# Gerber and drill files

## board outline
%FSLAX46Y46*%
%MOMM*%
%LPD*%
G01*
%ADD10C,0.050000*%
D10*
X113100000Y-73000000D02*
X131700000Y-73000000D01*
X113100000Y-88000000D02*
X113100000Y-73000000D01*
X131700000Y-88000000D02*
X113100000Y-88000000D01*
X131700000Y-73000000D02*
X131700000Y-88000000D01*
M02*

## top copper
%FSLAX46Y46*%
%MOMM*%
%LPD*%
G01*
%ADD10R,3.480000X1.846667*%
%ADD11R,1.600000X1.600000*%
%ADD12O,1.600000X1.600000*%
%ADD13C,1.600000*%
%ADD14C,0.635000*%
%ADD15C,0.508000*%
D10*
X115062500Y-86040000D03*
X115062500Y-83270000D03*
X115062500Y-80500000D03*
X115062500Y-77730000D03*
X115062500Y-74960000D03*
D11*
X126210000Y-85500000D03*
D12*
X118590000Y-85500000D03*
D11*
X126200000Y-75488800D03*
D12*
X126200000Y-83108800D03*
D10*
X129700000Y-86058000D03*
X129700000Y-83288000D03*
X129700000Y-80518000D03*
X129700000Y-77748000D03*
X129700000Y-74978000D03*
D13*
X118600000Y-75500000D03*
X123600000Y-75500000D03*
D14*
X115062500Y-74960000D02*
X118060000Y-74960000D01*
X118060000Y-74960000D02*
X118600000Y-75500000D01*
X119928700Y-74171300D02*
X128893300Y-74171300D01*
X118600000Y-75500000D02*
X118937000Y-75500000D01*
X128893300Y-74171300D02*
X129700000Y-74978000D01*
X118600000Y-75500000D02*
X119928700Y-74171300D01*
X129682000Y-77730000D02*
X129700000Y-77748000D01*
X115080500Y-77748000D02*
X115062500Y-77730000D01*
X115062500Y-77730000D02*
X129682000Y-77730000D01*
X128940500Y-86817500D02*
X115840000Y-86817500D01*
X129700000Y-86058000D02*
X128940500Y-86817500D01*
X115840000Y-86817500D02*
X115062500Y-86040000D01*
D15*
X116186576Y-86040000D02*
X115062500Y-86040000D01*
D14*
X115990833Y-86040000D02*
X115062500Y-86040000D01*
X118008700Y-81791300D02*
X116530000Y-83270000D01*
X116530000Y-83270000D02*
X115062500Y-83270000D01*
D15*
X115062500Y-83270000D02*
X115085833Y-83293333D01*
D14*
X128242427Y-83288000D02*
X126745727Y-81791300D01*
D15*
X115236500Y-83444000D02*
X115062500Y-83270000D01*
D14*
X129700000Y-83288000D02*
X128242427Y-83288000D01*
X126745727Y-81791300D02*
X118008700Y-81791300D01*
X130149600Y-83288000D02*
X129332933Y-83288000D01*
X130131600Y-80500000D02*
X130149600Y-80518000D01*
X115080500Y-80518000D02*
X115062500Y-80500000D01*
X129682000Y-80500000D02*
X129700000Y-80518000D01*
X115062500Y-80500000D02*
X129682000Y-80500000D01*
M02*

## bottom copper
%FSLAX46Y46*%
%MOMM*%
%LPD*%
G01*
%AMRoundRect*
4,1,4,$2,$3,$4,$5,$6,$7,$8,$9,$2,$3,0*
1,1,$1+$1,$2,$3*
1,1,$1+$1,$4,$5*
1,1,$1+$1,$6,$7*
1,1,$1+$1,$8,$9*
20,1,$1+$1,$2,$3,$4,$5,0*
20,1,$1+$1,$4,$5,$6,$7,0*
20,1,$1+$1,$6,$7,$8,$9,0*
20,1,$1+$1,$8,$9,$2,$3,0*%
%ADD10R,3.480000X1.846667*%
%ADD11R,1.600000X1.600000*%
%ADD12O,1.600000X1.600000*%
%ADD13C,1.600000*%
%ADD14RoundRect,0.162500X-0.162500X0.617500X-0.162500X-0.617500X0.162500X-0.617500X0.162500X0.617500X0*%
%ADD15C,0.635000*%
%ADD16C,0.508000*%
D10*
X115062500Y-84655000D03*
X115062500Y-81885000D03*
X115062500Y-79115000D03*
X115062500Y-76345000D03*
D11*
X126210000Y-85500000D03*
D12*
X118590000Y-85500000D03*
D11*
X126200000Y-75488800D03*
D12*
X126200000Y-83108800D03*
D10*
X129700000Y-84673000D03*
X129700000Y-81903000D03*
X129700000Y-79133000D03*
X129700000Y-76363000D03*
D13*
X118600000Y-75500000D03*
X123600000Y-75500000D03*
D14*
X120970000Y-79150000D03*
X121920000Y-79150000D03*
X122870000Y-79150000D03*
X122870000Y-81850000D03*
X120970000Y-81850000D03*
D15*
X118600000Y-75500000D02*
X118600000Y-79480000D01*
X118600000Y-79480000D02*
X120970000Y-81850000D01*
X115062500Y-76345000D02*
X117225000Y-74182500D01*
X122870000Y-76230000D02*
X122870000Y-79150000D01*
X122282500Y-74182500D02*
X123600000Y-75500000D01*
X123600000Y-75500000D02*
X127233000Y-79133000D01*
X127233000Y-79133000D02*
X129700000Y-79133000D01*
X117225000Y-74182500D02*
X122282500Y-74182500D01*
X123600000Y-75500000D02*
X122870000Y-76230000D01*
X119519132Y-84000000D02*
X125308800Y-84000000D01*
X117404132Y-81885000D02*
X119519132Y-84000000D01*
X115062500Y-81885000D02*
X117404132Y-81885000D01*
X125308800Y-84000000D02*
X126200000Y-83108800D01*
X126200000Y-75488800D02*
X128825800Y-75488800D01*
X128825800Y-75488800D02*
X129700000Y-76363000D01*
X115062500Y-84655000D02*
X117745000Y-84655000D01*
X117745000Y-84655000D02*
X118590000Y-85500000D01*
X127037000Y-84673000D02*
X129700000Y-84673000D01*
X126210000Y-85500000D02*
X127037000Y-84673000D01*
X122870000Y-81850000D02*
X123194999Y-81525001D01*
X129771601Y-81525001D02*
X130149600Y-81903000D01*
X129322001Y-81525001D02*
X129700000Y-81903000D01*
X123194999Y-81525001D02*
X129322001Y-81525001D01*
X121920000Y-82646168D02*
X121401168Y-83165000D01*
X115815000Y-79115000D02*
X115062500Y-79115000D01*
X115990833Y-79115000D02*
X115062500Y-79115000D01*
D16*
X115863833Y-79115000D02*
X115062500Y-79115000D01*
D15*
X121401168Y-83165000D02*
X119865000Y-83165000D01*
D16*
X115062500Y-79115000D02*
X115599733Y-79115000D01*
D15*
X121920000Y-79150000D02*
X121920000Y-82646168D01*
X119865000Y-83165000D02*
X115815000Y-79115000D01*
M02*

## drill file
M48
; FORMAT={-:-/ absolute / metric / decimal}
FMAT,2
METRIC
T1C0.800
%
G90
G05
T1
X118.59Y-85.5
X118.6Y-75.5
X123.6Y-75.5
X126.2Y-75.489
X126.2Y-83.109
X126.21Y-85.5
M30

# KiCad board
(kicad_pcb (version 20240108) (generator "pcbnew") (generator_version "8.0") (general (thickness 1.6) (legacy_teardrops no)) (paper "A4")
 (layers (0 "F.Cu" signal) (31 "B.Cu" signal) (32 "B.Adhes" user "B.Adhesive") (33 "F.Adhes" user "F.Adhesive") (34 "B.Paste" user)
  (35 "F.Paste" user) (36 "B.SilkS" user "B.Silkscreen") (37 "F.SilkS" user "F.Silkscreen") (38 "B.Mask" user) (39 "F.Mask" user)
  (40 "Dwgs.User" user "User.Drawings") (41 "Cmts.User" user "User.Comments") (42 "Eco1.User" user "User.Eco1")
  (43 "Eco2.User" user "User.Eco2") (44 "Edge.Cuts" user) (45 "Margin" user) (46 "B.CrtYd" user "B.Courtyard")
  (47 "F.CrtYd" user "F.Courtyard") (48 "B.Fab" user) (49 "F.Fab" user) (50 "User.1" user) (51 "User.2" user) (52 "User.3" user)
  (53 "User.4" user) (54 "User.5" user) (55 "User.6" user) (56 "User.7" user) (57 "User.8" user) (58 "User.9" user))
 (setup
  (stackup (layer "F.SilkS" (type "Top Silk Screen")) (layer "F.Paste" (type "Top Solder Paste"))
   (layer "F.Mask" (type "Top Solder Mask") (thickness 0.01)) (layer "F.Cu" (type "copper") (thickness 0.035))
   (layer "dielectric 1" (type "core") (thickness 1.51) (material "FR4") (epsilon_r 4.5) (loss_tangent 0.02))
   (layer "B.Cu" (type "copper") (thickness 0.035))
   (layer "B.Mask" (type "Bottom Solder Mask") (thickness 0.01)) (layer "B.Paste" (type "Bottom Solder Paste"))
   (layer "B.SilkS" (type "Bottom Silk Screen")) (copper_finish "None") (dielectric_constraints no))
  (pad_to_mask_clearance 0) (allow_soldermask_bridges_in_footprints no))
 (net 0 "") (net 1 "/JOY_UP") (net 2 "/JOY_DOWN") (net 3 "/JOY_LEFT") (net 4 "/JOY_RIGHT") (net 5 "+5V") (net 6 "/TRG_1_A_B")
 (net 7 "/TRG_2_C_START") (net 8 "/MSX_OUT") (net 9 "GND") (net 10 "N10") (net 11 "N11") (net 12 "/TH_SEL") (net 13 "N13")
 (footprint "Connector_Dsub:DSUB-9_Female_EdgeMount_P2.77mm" (layer "F.Cu") (at 115.0625 80.5 -90)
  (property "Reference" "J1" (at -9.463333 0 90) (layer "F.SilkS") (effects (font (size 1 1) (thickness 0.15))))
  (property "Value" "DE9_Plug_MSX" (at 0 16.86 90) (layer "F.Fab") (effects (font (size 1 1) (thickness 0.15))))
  (pad "1" smd rect (at 5.54 0 270) (size 1.846667 3.48) (layers "F.Cu" "F.Paste" "F.Mask") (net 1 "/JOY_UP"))
  (pad "2" smd rect (at 2.77 0 270) (size 1.846667 3.48) (layers "F.Cu" "F.Paste" "F.Mask") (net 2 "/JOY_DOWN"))
  (pad "3" smd rect (at 0 0 270) (size 1.846667 3.48) (layers "F.Cu" "F.Paste" "F.Mask") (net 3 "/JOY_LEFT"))
  (pad "4" smd rect (at -2.77 0 270) (size 1.846667 3.48) (layers "F.Cu" "F.Paste" "F.Mask") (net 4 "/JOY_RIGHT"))
  (pad "5" smd rect (at -5.54 0 270) (size 1.846667 3.48) (layers "F.Cu" "F.Paste" "F.Mask") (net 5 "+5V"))
  (pad "6" smd rect (at 4.155 0 270) (size 1.846667 3.48) (layers "B.Cu" "B.Paste" "B.Mask") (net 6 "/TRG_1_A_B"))
  (pad "7" smd rect (at 1.385 0 270) (size 1.846667 3.48) (layers "B.Cu" "B.Paste" "B.Mask") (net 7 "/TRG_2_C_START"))
  (pad "8" smd rect (at -1.385 0 270) (size 1.846667 3.48) (layers "B.Cu" "B.Paste" "B.Mask") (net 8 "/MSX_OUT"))
  (pad "9" smd rect (at -4.155 0 270) (size 1.846667 3.48) (layers "B.Cu" "B.Paste" "B.Mask") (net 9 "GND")))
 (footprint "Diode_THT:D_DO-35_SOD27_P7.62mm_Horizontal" (layer "F.Cu") (at 126.21 85.5 180)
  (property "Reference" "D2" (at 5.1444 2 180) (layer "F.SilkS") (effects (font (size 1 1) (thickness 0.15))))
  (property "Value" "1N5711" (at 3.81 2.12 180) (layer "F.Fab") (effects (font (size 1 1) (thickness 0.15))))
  (pad "1" thru_hole rect (at 0 0 180) (size 1.6 1.6) (drill 0.8) (layers "*.Cu" "*.Mask") (remove_unused_layers no) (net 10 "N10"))
  (pad "2" thru_hole oval (at 7.62 0 180) (size 1.6 1.6) (drill 0.8) (layers "*.Cu" "*.Mask") (remove_unused_layers no) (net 6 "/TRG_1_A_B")))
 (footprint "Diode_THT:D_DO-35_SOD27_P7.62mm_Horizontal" (layer "F.Cu") (at 126.2 75.4888 -90)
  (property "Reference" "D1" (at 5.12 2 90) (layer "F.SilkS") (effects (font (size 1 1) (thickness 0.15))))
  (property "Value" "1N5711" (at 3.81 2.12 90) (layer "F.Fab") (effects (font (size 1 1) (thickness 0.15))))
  (pad "1" thru_hole rect (at 0 0 270) (size 1.6 1.6) (drill 0.8) (layers "*.Cu" "*.Mask") (remove_unused_layers no) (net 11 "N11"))
  (pad "2" thru_hole oval (at 7.62 0 270) (size 1.6 1.6) (drill 0.8) (layers "*.Cu" "*.Mask") (remove_unused_layers no)
   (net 7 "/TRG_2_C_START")))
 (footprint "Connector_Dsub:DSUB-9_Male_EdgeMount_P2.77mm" (layer "F.Cu") (at 129.7 80.518 90)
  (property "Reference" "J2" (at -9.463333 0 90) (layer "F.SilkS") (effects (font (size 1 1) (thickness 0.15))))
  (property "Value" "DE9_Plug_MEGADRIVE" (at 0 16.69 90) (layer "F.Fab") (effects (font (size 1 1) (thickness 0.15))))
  (pad "1" smd rect (at -5.54 0 90) (size 1.846667 3.48) (layers "F.Cu" "F.Paste" "F.Mask") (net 1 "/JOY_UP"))
  (pad "2" smd rect (at -2.77 0 90) (size 1.846667 3.48) (layers "F.Cu" "F.Paste" "F.Mask") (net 2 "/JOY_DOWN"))
  (pad "3" smd rect (at 0 0 90) (size 1.846667 3.48) (layers "F.Cu" "F.Paste" "F.Mask") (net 3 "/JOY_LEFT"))
  (pad "4" smd rect (at 2.77 0 90) (size 1.846667 3.48) (layers "F.Cu" "F.Paste" "F.Mask") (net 4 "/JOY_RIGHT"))
  (pad "5" smd rect (at 5.54 0 90) (size 1.846667 3.48) (layers "F.Cu" "F.Paste" "F.Mask") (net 5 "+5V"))
  (pad "6" smd rect (at -4.155 0 90) (size 1.846667 3.48) (layers "B.Cu" "B.Paste" "B.Mask") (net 10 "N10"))
  (pad "7" smd rect (at -1.385 0 90) (size 1.846667 3.48) (layers "B.Cu" "B.Paste" "B.Mask") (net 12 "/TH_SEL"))
  (pad "8" smd rect (at 1.385 0 90) (size 1.846667 3.48) (layers "B.Cu" "B.Paste" "B.Mask") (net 9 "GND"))
  (pad "9" smd rect (at 4.155 0 90) (size 1.846667 3.48) (layers "B.Cu" "B.Paste" "B.Mask") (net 11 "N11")))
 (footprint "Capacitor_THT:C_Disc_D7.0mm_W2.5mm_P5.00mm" (layer "F.Cu") (at 118.6 75.5)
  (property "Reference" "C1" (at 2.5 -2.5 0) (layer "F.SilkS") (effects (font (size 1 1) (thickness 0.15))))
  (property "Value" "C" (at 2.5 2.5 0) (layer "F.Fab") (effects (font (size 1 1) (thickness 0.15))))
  (pad "1" thru_hole circle (at 0 0) (size 1.6 1.6) (drill 0.8) (layers "*.Cu" "*.Mask") (remove_unused_layers no) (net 5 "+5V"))
  (pad "2" thru_hole circle (at 5 0) (size 1.6 1.6) (drill 0.8) (layers "*.Cu" "*.Mask") (remove_unused_layers no) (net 9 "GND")))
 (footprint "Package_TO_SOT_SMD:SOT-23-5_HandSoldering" (layer "B.Cu") (at 121.92 80.5 -90)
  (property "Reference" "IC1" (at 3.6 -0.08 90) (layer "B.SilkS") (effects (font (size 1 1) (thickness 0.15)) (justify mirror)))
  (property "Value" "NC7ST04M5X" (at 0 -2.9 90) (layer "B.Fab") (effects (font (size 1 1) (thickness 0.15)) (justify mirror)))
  (pad "1" smd roundrect (at -1.35 0.95 270) (size 1.56 0.65) (layers "B.Cu" "B.Paste" "B.Mask") (roundrect_rratio 0.25) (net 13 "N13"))
  (pad "2" smd roundrect (at -1.35 0 270) (size 1.56 0.65) (layers "B.Cu" "B.Paste" "B.Mask") (roundrect_rratio 0.25) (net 8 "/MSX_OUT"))
  (pad "3" smd roundrect (at -1.35 -0.95 270) (size 1.56 0.65) (layers "B.Cu" "B.Paste" "B.Mask") (roundrect_rratio 0.25) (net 9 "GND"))
  (pad "4" smd roundrect (at 1.35 -0.95 270) (size 1.56 0.65) (layers "B.Cu" "B.Paste" "B.Mask") (roundrect_rratio 0.25) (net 12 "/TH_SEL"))
  (pad "5" smd roundrect (at 1.35 0.95 270) (size 1.56 0.65) (layers "B.Cu" "B.Paste" "B.Mask") (roundrect_rratio 0.25) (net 5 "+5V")))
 (gr_line (start 113.1 73) (end 131.7 73) (stroke (width 0.05) (type default)) (layer "Edge.Cuts"))
 (gr_line (start 113.1 88) (end 113.1 73) (stroke (width 0.05) (type default)) (layer "Edge.Cuts"))
 (gr_line (start 131.7 88) (end 113.1 88) (stroke (width 0.05) (type default)) (layer "Edge.Cuts"))
 (gr_line (start 131.7 73) (end 131.7 88) (stroke (width 0.05) (type default)) (layer "Edge.Cuts"))
 (segment (start 115.0625 74.96) (end 118.06 74.96) (width 0.635) (layer "F.Cu") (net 5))
 (segment (start 118.06 74.96) (end 118.6 75.5) (width 0.635) (layer "F.Cu") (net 5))
 (segment (start 119.9287 74.1713) (end 128.8933 74.1713) (width 0.635) (layer "F.Cu") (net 5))
 (segment (start 118.6 75.5) (end 118.937 75.5) (width 0.635) (layer "F.Cu") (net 5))
 (segment (start 128.8933 74.1713) (end 129.7 74.978) (width 0.635) (layer "F.Cu") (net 5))
 (segment (start 118.6 75.5) (end 119.9287 74.1713) (width 0.635) (layer "F.Cu") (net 5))
 (segment (start 118.6 75.5) (end 118.6 79.48) (width 0.635) (layer "B.Cu") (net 5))
 (segment (start 118.6 79.48) (end 120.97 81.85) (width 0.635) (layer "B.Cu") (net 5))
 (segment (start 115.0625 76.345) (end 117.225 74.1825) (width 0.635) (layer "B.Cu") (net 9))
 (segment (start 122.87 76.23) (end 122.87 79.15) (width 0.635) (layer "B.Cu") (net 9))
 (segment (start 122.2825 74.1825) (end 123.6 75.5) (width 0.635) (layer "B.Cu") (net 9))
 (segment (start 123.6 75.5) (end 127.233 79.133) (width 0.635) (layer "B.Cu") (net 9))
 (segment (start 127.233 79.133) (end 129.7 79.133) (width 0.635) (layer "B.Cu") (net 9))
 (segment (start 117.225 74.1825) (end 122.2825 74.1825) (width 0.635) (layer "B.Cu") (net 9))
 (segment (start 123.6 75.5) (end 122.87 76.23) (width 0.635) (layer "B.Cu") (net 9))
 (segment (start 119.519132 84) (end 125.3088 84) (width 0.635) (layer "B.Cu") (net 7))
 (segment (start 117.404132 81.885) (end 119.519132 84) (width 0.635) (layer "B.Cu") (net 7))
 (segment (start 115.0625 81.885) (end 117.404132 81.885) (width 0.635) (layer "B.Cu") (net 7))
 (segment (start 125.3088 84) (end 126.2 83.1088) (width 0.635) (layer "B.Cu") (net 7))
 (segment (start 126.2 75.4888) (end 128.8258 75.4888) (width 0.635) (layer "B.Cu") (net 11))
 (segment (start 128.8258 75.4888) (end 129.7 76.363) (width 0.635) (layer "B.Cu") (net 11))
 (segment (start 115.0625 84.655) (end 117.745 84.655) (width 0.635) (layer "B.Cu") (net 6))
 (segment (start 117.745 84.655) (end 118.59 85.5) (width 0.635) (layer "B.Cu") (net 6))
 (segment (start 127.037 84.673) (end 129.7 84.673) (width 0.635) (layer "B.Cu") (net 10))
 (segment (start 126.21 85.5) (end 127.037 84.673) (width 0.635) (layer "B.Cu") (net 10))
 (segment (start 122.87 81.85) (end 123.194999 81.525001) (width 0.635) (layer "B.Cu") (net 12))
 (segment (start 129.771601 81.525001) (end 130.1496 81.903) (width 0.635) (layer "B.Cu") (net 12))
 (segment (start 129.322001 81.525001) (end 129.7 81.903) (width 0.635) (layer "B.Cu") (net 12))
 (segment (start 123.194999 81.525001) (end 129.322001 81.525001) (width 0.635) (layer "B.Cu") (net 12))
 (segment (start 121.92 82.646168) (end 121.401168 83.165) (width 0.635) (layer "B.Cu") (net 8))
 (segment (start 115.815 79.115) (end 115.0625 79.115) (width 0.635) (layer "B.Cu") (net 8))
 (segment (start 115.990833 79.115) (end 115.0625 79.115) (width 0.635) (layer "B.Cu") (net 8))
 (segment (start 115.863833 79.115) (end 115.0625 79.115) (width 0.508) (layer "B.Cu") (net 8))
 (segment (start 121.401168 83.165) (end 119.865 83.165) (width 0.635) (layer "B.Cu") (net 8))
 (segment (start 115.0625 79.115) (end 115.599733 79.115) (width 0.508) (layer "B.Cu") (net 8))
 (segment (start 121.92 79.15) (end 121.92 82.646168) (width 0.635) (layer "B.Cu") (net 8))
 (segment (start 119.865 83.165) (end 115.815 79.115) (width 0.635) (layer "B.Cu") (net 8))
 (segment (start 129.682 77.73) (end 129.7 77.748) (width 0.635) (layer "F.Cu") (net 4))
 (segment (start 115.0805 77.748) (end 115.0625 77.73) (width 0.635) (layer "F.Cu") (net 4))
 (segment (start 115.0625 77.73) (end 129.682 77.73) (width 0.635) (layer "F.Cu") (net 4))
 (segment (start 128.9405 86.8175) (end 115.84 86.8175) (width 0.635) (layer "F.Cu") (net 1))
 (segment (start 129.7 86.058) (end 128.9405 86.8175) (width 0.635) (layer "F.Cu") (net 1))
 (segment (start 115.84 86.8175) (end 115.0625 86.04) (width 0.635) (layer "F.Cu") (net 1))
 (segment (start 116.186576 86.04) (end 115.0625 86.04) (width 0.508) (layer "F.Cu") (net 1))
 (segment (start 115.990833 86.04) (end 115.0625 86.04) (width 0.635) (layer "F.Cu") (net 1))
 (segment (start 118.0087 81.7913) (end 116.53 83.27) (width 0.635) (layer "F.Cu") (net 2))
 (segment (start 116.53 83.27) (end 115.0625 83.27) (width 0.635) (layer "F.Cu") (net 2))
 (segment (start 115.0625 83.27) (end 115.085833 83.293333) (width 0.508) (layer "F.Cu") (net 2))
 (segment (start 128.242427 83.288) (end 126.745727 81.7913) (width 0.635) (layer "F.Cu") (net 2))
 (segment (start 115.2365 83.444) (end 115.0625 83.27) (width 0.508) (layer "F.Cu") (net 2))
 (segment (start 129.7 83.288) (end 128.242427 83.288) (width 0.635) (layer "F.Cu") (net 2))
 (segment (start 126.745727 81.7913) (end 118.0087 81.7913) (width 0.635) (layer "F.Cu") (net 2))
 (segment (start 130.1496 83.288) (end 129.332933 83.288) (width 0.635) (layer "F.Cu") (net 2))
 (segment (start 130.1316 80.5) (end 130.1496 80.518) (width 0.635) (layer "F.Cu") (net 3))
 (segment (start 115.0805 80.518) (end 115.0625 80.5) (width 0.635) (layer "F.Cu") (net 3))
 (segment (start 129.682 80.5) (end 129.7 80.518) (width 0.635) (layer "F.Cu") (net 3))
 (segment (start 115.0625 80.5) (end 129.682 80.5) (width 0.635) (layer "F.Cu") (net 3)))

